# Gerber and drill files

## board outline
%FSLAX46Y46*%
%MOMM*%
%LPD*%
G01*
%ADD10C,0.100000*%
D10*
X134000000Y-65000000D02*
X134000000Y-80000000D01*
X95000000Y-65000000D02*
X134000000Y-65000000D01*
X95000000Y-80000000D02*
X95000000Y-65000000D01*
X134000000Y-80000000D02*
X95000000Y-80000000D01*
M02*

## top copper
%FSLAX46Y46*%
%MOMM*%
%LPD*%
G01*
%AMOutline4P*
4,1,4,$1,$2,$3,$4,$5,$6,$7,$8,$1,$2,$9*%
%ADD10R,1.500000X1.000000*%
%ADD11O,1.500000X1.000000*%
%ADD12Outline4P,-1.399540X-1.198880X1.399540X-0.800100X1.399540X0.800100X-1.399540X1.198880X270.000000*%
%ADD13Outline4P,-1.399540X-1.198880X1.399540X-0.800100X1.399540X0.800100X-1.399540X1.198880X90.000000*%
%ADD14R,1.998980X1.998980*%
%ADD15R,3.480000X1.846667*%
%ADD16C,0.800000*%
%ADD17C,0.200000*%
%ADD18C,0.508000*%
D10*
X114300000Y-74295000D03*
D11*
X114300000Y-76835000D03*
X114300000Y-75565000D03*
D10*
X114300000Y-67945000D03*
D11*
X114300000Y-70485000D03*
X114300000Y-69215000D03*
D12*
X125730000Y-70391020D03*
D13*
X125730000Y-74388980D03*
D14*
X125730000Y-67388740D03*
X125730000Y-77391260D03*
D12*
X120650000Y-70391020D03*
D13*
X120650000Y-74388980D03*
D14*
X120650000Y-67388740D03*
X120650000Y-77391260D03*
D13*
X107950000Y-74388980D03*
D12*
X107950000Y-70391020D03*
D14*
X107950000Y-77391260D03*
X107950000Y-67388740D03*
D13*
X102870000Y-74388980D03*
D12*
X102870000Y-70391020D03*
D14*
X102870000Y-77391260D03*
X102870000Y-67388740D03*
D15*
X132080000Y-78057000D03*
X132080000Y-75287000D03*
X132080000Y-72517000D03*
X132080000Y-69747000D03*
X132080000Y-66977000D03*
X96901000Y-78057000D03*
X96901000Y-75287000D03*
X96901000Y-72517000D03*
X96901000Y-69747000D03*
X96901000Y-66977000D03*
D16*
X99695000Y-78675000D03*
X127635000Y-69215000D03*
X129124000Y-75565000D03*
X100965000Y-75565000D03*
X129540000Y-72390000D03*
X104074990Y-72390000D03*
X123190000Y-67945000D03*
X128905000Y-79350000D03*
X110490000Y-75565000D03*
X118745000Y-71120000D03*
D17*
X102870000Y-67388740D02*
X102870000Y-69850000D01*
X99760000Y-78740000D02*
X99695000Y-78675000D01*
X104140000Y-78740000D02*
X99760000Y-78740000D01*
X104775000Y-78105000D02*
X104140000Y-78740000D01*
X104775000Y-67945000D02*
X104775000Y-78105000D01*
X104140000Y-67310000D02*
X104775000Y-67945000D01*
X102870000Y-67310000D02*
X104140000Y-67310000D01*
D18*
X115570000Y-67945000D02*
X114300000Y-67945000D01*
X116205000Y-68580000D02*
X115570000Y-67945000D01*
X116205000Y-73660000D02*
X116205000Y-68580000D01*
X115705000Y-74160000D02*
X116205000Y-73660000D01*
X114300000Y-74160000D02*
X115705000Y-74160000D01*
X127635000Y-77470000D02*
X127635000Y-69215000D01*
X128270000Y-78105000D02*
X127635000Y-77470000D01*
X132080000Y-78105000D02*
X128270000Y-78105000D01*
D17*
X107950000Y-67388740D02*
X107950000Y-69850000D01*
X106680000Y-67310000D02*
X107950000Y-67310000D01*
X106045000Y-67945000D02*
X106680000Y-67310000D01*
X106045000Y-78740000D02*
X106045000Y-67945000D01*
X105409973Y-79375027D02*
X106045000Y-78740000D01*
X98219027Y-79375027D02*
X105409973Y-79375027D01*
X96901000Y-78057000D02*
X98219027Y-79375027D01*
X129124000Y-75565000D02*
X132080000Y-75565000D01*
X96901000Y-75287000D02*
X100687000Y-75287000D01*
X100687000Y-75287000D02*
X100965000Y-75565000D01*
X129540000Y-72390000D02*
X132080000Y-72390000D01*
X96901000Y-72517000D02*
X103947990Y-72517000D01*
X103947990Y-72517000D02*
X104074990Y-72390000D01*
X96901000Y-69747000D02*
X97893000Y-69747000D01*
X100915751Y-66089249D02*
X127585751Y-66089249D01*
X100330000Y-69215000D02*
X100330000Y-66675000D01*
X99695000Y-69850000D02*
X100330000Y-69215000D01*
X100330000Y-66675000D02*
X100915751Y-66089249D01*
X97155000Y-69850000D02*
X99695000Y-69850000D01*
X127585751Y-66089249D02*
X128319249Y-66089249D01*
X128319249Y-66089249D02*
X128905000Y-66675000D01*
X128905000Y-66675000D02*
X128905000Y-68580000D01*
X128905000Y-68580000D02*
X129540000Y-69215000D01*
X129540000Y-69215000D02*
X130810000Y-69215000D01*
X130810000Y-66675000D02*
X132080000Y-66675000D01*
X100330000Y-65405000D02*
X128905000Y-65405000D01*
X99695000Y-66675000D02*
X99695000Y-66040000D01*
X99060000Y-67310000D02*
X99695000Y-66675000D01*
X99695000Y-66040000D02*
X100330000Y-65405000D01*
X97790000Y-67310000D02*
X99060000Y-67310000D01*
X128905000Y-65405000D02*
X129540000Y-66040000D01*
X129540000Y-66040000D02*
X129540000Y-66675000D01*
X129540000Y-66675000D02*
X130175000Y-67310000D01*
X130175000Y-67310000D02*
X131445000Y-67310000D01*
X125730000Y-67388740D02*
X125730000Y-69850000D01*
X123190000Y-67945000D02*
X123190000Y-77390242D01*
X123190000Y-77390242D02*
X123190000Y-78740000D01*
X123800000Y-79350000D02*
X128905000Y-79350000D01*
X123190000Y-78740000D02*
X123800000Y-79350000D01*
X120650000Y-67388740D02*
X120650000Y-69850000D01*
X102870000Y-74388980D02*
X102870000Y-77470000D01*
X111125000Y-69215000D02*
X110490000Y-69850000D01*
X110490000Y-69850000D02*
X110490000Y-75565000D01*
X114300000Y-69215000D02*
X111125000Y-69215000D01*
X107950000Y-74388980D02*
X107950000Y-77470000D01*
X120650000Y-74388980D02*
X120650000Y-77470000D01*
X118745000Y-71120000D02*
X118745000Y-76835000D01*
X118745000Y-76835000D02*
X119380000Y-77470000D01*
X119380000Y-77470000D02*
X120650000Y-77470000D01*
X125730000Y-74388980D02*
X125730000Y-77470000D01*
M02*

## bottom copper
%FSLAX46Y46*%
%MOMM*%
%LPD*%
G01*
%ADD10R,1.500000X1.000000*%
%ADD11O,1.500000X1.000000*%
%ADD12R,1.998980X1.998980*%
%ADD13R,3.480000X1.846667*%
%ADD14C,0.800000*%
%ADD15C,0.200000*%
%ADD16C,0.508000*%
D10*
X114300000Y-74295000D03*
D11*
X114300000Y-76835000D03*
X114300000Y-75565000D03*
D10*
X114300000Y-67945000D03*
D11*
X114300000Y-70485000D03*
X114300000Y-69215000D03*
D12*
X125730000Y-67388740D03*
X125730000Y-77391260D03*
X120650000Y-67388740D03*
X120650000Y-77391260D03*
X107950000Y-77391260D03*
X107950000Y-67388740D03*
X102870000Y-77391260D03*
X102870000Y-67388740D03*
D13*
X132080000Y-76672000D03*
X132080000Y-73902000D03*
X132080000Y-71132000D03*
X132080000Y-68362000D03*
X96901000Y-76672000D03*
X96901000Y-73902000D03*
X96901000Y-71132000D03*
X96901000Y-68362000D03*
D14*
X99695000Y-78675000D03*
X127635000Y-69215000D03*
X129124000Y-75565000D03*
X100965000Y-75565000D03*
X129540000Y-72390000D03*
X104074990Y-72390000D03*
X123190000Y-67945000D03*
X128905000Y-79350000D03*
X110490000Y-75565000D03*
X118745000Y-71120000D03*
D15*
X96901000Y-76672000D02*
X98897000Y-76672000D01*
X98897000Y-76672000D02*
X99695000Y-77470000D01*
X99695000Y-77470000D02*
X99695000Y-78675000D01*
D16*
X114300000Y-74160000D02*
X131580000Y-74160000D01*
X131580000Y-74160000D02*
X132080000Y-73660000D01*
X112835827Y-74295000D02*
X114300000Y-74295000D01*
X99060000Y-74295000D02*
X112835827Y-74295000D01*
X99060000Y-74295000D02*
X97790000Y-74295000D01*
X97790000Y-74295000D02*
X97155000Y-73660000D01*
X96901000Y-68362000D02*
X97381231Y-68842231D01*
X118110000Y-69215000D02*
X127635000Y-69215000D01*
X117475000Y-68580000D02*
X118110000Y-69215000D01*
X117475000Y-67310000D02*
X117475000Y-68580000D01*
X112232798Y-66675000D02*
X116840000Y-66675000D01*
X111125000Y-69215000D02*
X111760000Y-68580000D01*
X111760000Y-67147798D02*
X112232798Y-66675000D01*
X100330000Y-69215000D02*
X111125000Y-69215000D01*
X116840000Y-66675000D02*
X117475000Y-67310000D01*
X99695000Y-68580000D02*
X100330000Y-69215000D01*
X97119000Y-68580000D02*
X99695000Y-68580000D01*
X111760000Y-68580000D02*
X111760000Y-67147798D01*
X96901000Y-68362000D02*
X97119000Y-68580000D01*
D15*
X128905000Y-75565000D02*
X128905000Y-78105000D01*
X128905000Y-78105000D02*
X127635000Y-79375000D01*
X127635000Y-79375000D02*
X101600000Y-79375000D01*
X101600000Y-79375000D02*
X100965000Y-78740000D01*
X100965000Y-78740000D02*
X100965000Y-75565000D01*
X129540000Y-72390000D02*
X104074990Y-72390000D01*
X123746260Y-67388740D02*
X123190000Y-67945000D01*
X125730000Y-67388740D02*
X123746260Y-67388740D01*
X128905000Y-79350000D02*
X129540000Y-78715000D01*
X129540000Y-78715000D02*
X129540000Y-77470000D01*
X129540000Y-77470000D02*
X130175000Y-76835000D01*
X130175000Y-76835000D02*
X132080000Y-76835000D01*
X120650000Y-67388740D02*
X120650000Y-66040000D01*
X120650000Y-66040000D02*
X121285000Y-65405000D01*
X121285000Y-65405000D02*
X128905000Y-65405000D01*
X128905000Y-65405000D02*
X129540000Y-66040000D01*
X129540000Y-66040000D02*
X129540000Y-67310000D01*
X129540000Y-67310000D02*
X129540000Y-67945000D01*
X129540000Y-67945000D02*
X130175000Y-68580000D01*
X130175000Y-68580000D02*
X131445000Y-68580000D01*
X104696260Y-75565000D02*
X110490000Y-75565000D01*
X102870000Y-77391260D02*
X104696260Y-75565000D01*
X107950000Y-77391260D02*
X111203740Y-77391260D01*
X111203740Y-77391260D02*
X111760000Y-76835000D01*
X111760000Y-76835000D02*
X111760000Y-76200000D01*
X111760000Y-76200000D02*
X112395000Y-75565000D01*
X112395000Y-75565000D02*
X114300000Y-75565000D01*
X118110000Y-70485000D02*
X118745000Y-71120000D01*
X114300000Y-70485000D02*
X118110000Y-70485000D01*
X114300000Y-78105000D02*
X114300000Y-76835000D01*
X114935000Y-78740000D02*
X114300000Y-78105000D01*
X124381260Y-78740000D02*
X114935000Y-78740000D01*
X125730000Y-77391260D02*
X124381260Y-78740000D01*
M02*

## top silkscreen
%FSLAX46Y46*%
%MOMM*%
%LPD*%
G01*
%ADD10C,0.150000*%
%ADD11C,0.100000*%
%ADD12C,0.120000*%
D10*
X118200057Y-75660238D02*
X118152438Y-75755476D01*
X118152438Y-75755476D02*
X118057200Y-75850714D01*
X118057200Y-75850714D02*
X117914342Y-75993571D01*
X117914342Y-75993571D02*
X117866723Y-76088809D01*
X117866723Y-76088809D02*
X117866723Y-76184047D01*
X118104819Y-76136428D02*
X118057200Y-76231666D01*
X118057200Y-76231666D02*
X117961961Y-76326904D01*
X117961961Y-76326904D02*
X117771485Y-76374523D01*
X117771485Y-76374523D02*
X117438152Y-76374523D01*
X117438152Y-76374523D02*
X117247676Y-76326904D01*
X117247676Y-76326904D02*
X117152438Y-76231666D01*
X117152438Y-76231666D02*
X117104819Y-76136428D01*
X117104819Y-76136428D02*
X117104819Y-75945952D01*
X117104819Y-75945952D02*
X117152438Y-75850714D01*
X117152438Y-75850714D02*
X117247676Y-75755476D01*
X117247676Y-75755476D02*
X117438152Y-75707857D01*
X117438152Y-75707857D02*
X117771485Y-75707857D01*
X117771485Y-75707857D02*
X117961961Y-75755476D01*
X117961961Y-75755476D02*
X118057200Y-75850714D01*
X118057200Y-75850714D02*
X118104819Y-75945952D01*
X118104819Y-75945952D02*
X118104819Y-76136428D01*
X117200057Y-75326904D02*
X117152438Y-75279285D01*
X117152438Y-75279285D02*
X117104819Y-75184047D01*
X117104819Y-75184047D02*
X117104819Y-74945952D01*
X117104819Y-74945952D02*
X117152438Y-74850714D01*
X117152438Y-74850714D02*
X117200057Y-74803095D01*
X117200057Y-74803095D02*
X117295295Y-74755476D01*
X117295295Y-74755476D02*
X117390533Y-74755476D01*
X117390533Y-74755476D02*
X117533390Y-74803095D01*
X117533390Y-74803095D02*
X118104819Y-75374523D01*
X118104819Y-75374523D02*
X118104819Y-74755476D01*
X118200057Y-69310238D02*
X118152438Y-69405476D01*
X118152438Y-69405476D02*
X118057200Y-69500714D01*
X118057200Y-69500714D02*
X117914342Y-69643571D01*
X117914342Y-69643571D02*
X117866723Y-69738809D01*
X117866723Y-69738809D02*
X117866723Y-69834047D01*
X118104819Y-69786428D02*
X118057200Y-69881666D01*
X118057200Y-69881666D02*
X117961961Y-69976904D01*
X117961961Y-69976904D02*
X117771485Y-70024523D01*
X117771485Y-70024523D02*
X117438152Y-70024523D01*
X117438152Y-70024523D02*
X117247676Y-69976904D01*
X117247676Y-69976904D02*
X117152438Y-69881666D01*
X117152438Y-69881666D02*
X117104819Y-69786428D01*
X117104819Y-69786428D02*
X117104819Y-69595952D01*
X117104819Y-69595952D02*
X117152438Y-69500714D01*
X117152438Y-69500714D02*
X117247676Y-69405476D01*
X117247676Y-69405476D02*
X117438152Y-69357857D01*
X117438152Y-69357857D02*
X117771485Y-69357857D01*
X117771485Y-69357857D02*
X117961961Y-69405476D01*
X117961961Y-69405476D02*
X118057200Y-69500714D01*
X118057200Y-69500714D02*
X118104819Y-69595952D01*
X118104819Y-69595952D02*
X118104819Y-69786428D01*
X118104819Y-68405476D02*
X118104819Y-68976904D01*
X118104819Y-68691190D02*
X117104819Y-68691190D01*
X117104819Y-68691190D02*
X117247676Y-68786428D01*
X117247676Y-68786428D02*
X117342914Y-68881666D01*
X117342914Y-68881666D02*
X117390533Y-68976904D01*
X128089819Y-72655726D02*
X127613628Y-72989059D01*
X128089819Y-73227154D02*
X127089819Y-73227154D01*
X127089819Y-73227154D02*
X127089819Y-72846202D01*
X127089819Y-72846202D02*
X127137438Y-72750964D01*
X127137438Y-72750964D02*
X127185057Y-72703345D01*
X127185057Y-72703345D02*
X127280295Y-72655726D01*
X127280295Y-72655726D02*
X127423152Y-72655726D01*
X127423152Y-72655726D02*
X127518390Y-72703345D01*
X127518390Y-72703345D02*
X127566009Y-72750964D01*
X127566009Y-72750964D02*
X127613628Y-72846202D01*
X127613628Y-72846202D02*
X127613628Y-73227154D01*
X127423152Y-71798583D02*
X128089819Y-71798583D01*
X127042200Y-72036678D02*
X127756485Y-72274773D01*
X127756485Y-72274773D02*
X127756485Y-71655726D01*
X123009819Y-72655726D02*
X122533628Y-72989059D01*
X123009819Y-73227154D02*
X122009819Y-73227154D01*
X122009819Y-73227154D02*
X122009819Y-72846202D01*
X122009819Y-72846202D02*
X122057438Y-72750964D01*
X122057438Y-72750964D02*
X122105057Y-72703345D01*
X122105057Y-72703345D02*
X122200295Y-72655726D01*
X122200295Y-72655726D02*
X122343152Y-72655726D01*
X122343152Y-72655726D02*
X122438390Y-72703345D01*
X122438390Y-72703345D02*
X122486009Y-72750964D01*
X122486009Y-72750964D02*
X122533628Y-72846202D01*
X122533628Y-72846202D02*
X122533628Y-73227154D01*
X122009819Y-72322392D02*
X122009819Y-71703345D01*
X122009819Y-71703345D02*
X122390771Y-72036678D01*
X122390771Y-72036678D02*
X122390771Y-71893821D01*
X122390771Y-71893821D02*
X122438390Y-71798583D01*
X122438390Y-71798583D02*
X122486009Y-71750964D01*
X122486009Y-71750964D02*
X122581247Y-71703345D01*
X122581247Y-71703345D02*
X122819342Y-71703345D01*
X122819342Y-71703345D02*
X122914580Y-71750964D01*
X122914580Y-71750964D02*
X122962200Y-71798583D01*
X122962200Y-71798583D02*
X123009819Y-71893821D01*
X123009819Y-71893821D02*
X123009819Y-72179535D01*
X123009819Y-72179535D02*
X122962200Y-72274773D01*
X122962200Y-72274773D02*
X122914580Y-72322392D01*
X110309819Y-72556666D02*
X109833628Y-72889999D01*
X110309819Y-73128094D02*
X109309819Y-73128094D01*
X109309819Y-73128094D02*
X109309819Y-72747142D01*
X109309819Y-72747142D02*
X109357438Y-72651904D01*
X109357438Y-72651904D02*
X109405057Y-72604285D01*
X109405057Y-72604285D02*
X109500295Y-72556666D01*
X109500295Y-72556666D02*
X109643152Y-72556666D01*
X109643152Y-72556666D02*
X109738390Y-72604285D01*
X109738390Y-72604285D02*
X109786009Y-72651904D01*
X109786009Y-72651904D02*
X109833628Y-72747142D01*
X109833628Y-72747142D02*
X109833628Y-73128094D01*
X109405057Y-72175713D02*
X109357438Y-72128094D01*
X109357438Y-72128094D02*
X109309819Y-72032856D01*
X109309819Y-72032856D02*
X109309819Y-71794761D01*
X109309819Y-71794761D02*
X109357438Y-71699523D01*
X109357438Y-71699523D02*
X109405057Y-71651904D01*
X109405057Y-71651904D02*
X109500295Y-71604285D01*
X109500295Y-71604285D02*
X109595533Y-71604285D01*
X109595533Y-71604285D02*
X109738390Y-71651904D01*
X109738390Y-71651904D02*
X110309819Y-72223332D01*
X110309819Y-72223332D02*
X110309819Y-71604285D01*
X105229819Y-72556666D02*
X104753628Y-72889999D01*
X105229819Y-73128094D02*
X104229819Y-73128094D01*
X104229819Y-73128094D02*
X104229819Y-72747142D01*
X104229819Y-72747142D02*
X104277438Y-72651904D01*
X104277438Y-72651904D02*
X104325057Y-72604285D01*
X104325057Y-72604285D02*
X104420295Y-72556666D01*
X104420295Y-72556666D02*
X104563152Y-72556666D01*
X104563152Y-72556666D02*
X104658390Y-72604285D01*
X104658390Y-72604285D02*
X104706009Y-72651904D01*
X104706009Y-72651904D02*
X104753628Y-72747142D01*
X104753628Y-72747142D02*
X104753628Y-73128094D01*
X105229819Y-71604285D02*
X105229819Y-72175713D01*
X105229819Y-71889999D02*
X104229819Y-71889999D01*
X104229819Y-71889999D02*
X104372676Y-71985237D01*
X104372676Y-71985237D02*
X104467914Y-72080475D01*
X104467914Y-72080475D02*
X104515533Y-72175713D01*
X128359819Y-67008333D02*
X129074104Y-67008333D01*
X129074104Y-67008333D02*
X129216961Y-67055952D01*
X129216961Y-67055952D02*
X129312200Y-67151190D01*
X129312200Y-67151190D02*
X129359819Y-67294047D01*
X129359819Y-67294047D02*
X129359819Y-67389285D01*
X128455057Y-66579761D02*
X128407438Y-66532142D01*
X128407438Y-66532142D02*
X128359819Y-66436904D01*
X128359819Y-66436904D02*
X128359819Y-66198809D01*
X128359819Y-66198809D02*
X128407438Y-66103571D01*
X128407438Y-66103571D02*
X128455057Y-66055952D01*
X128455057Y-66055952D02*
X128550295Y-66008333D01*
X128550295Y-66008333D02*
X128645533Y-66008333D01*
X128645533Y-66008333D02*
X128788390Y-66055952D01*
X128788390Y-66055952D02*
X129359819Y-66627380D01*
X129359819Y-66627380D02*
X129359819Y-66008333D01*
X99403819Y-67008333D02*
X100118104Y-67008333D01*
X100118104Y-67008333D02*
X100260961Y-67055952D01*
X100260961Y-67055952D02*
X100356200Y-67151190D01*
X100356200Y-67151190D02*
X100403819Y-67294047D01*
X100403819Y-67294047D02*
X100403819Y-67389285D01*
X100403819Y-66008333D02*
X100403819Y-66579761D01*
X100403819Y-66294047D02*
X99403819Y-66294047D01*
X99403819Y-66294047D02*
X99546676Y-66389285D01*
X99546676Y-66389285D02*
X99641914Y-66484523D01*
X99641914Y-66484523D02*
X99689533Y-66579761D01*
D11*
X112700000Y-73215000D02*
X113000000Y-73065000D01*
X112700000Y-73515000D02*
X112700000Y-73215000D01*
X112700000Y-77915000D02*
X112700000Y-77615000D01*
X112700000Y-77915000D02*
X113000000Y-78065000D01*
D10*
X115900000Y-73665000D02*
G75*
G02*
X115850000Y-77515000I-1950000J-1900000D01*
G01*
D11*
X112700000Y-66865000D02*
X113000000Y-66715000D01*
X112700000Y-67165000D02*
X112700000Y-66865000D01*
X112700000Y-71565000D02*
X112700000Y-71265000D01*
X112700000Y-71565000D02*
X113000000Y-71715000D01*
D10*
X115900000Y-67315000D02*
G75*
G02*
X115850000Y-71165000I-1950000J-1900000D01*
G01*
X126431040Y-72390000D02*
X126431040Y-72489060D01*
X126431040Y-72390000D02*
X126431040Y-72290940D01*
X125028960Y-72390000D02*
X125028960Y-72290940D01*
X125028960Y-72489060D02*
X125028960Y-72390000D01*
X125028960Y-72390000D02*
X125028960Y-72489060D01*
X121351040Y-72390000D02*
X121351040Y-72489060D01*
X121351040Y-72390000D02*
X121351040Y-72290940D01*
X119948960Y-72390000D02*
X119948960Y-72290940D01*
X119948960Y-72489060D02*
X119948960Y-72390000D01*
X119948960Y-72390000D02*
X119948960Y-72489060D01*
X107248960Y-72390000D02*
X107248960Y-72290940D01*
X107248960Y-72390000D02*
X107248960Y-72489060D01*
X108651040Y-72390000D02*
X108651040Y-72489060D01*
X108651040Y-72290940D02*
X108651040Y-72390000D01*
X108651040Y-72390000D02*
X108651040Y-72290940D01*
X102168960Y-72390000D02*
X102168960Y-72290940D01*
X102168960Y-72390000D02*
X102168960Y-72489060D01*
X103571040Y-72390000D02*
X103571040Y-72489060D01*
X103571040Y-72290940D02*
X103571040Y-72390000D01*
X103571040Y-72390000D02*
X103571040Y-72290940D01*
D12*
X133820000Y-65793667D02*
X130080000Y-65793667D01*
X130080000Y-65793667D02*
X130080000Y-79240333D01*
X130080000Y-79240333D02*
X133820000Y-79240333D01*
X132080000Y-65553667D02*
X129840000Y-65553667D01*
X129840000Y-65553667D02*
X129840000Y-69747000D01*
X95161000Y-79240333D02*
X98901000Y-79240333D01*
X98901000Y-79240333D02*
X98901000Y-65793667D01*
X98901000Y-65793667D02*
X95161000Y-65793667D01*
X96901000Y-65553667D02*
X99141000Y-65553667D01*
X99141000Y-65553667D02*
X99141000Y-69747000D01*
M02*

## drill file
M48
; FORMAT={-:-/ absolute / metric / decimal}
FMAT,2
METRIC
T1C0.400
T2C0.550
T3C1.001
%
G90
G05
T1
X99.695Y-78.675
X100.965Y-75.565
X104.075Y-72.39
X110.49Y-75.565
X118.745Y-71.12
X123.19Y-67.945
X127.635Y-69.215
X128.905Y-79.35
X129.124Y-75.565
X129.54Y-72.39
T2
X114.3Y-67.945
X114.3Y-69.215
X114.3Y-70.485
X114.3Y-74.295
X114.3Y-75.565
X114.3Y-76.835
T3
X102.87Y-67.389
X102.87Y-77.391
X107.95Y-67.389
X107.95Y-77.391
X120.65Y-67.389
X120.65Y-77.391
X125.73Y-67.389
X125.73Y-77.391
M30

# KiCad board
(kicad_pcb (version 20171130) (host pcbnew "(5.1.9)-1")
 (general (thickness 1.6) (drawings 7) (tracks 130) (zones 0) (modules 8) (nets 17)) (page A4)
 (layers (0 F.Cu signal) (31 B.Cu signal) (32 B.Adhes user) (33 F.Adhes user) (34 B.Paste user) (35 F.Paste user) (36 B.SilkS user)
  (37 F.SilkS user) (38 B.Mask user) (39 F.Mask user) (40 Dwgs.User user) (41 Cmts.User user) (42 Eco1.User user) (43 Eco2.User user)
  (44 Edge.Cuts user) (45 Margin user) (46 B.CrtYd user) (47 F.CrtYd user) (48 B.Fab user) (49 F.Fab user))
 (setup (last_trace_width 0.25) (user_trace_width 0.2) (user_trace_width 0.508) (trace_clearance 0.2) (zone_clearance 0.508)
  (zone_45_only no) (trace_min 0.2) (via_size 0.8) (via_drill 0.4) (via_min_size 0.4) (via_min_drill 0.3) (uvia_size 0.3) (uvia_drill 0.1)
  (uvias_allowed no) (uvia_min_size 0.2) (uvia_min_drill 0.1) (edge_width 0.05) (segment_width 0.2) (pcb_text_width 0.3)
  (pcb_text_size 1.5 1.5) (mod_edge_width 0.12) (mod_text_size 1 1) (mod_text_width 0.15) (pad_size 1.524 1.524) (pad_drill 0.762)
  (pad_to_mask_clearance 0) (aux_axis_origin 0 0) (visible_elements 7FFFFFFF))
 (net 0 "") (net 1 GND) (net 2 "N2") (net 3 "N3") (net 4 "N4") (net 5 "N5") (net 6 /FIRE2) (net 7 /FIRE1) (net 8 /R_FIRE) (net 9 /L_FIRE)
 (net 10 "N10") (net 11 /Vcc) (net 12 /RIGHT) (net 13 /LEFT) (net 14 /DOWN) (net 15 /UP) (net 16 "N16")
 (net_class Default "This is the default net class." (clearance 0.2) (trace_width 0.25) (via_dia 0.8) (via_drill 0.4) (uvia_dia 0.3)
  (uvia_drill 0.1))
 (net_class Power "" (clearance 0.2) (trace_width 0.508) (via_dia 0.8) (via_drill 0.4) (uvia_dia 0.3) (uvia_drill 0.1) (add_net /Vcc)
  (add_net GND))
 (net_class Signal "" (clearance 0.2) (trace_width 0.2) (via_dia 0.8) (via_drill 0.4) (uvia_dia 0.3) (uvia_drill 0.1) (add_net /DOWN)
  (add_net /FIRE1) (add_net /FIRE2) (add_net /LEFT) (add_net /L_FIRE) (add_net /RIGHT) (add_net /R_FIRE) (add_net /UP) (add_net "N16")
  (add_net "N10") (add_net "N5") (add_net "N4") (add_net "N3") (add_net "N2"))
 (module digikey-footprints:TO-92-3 (layer F.Cu) (at 114.3 74.295 270)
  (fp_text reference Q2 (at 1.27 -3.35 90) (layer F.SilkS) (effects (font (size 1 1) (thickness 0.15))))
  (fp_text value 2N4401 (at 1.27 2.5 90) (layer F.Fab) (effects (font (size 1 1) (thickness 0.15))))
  (fp_line (start -1.08 1.6) (end -1.23 1.3) (layer F.SilkS) (width 0.1))
  (fp_line (start -0.78 1.6) (end -1.08 1.6) (layer F.SilkS) (width 0.1))
  (fp_line (start 3.62 1.6) (end 3.32 1.6) (layer F.SilkS) (width 0.1))
  (fp_line (start 3.62 1.6) (end 3.77 1.3) (layer F.SilkS) (width 0.1))
  (fp_arc (start 1.27 0.35) (end -0.63 -1.6) (angle 90) (layer F.SilkS) (width 0.15))
  (pad 1 thru_hole rect (at 0 0 90) (size 1 1.5) (drill 0.55) (layers *.Cu *.Mask) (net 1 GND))
  (pad 3 thru_hole oval (at 2.54 0 90) (size 1 1.5) (drill 0.55) (layers *.Cu *.Mask) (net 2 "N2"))
  (pad 2 thru_hole oval (at 1.27 0 90) (size 1 1.5) (drill 0.55) (layers *.Cu *.Mask) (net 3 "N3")))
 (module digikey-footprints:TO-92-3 (layer F.Cu) (at 114.3 67.945 270)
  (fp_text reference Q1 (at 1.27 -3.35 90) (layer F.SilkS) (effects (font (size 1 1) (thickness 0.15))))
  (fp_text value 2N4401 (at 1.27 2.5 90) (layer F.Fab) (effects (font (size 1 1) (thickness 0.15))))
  (fp_line (start -1.08 1.6) (end -1.23 1.3) (layer F.SilkS) (width 0.1))
  (fp_line (start -0.78 1.6) (end -1.08 1.6) (layer F.SilkS) (width 0.1))
  (fp_line (start 3.62 1.6) (end 3.32 1.6) (layer F.SilkS) (width 0.1))
  (fp_line (start 3.62 1.6) (end 3.77 1.3) (layer F.SilkS) (width 0.1))
  (fp_arc (start 1.27 0.35) (end -0.63 -1.6) (angle 90) (layer F.SilkS) (width 0.15))
  (pad 1 thru_hole rect (at 0 0 90) (size 1 1.5) (drill 0.55) (layers *.Cu *.Mask) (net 1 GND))
  (pad 3 thru_hole oval (at 2.54 0 90) (size 1 1.5) (drill 0.55) (layers *.Cu *.Mask) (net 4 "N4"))
  (pad 2 thru_hole oval (at 1.27 0 90) (size 1 1.5) (drill 0.55) (layers *.Cu *.Mask) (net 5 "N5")))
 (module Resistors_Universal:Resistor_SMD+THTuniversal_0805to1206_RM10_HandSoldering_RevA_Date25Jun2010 (layer F.Cu) (at 125.73 72.39 270)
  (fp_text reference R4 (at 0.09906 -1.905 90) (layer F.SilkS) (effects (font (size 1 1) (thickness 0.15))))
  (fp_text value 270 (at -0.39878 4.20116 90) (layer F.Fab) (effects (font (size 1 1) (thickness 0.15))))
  (fp_line (start 0 -0.70104) (end 0.09906 -0.70104) (layer F.SilkS) (width 0.15))
  (fp_line (start 0 -0.70104) (end -0.09906 -0.70104) (layer F.SilkS) (width 0.15))
  (fp_line (start 0 0.70104) (end -0.09906 0.70104) (layer F.SilkS) (width 0.15))
  (fp_line (start 0.09906 0.70104) (end 0 0.70104) (layer F.SilkS) (width 0.15))
  (fp_line (start 0 0.70104) (end 0.09906 0.70104) (layer F.SilkS) (width 0.15))
  (pad 1 smd trapezoid (at -1.99898 0 270) (size 2.79908 1.99898) (rect_delta 0.39878 0) (layers F.Cu F.Paste F.Mask) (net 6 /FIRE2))
  (pad 2 smd trapezoid (at 1.99898 0 90) (size 2.79908 1.99898) (rect_delta 0.39878 0) (layers F.Cu F.Paste F.Mask) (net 2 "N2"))
  (pad 1 thru_hole rect (at -5.00126 0 90) (size 1.99898 1.99898) (drill 1.00076) (layers *.Cu *.Mask) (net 6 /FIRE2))
  (pad 2 thru_hole rect (at 5.00126 0 90) (size 1.99898 1.99898) (drill 1.00076) (layers *.Cu *.Mask) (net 2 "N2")))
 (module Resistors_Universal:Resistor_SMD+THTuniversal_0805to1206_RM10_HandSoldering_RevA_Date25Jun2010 (layer F.Cu) (at 120.65 72.39 270)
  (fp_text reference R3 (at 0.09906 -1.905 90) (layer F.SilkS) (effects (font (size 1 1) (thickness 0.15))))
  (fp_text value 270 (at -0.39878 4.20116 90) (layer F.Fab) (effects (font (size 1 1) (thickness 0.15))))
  (fp_line (start 0 -0.70104) (end 0.09906 -0.70104) (layer F.SilkS) (width 0.15))
  (fp_line (start 0 -0.70104) (end -0.09906 -0.70104) (layer F.SilkS) (width 0.15))
  (fp_line (start 0 0.70104) (end -0.09906 0.70104) (layer F.SilkS) (width 0.15))
  (fp_line (start 0.09906 0.70104) (end 0 0.70104) (layer F.SilkS) (width 0.15))
  (fp_line (start 0 0.70104) (end 0.09906 0.70104) (layer F.SilkS) (width 0.15))
  (pad 1 smd trapezoid (at -1.99898 0 270) (size 2.79908 1.99898) (rect_delta 0.39878 0) (layers F.Cu F.Paste F.Mask) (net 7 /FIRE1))
  (pad 2 smd trapezoid (at 1.99898 0 90) (size 2.79908 1.99898) (rect_delta 0.39878 0) (layers F.Cu F.Paste F.Mask) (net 4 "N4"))
  (pad 1 thru_hole rect (at -5.00126 0 90) (size 1.99898 1.99898) (drill 1.00076) (layers *.Cu *.Mask) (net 7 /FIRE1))
  (pad 2 thru_hole rect (at 5.00126 0 90) (size 1.99898 1.99898) (drill 1.00076) (layers *.Cu *.Mask) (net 4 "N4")))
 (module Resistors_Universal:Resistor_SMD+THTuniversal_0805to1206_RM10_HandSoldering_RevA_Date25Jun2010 (layer F.Cu) (at 107.95 72.39 90)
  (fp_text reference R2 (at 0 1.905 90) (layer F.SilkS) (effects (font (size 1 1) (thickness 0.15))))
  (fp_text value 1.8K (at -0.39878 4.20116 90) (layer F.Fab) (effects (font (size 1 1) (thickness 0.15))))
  (fp_line (start 0 -0.70104) (end 0.09906 -0.70104) (layer F.SilkS) (width 0.15))
  (fp_line (start 0 -0.70104) (end -0.09906 -0.70104) (layer F.SilkS) (width 0.15))
  (fp_line (start 0 0.70104) (end -0.09906 0.70104) (layer F.SilkS) (width 0.15))
  (fp_line (start 0.09906 0.70104) (end 0 0.70104) (layer F.SilkS) (width 0.15))
  (fp_line (start 0 0.70104) (end 0.09906 0.70104) (layer F.SilkS) (width 0.15))
  (pad 1 smd trapezoid (at -1.99898 0 90) (size 2.79908 1.99898) (rect_delta 0.39878 0) (layers F.Cu F.Paste F.Mask) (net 3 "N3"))
  (pad 2 smd trapezoid (at 1.99898 0 270) (size 2.79908 1.99898) (rect_delta 0.39878 0) (layers F.Cu F.Paste F.Mask) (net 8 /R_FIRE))
  (pad 1 thru_hole rect (at -5.00126 0 270) (size 1.99898 1.99898) (drill 1.00076) (layers *.Cu *.Mask) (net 3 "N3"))
  (pad 2 thru_hole rect (at 5.00126 0 270) (size 1.99898 1.99898) (drill 1.00076) (layers *.Cu *.Mask) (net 8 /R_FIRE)))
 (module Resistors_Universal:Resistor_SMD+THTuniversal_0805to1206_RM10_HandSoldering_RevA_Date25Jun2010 (layer F.Cu) (at 102.87 72.39 90)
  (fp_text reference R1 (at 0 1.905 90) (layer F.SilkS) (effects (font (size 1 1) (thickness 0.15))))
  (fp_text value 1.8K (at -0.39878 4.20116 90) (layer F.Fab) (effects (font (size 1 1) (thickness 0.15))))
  (fp_line (start 0 -0.70104) (end 0.09906 -0.70104) (layer F.SilkS) (width 0.15))
  (fp_line (start 0 -0.70104) (end -0.09906 -0.70104) (layer F.SilkS) (width 0.15))
  (fp_line (start 0 0.70104) (end -0.09906 0.70104) (layer F.SilkS) (width 0.15))
  (fp_line (start 0.09906 0.70104) (end 0 0.70104) (layer F.SilkS) (width 0.15))
  (fp_line (start 0 0.70104) (end 0.09906 0.70104) (layer F.SilkS) (width 0.15))
  (pad 1 smd trapezoid (at -1.99898 0 90) (size 2.79908 1.99898) (rect_delta 0.39878 0) (layers F.Cu F.Paste F.Mask) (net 5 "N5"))
  (pad 2 smd trapezoid (at 1.99898 0 270) (size 2.79908 1.99898) (rect_delta 0.39878 0) (layers F.Cu F.Paste F.Mask) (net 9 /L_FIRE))
  (pad 1 thru_hole rect (at -5.00126 0 270) (size 1.99898 1.99898) (drill 1.00076) (layers *.Cu *.Mask) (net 5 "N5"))
  (pad 2 thru_hole rect (at 5.00126 0 270) (size 1.99898 1.99898) (drill 1.00076) (layers *.Cu *.Mask) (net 9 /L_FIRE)))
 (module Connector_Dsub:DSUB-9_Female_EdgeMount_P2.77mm (layer F.Cu) (at 132.08 72.517 90)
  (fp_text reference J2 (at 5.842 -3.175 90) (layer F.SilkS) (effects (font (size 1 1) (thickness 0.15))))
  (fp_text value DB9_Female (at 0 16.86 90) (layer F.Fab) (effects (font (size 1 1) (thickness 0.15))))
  (fp_line (start 6.723333 1.74) (end 6.723333 -2) (layer F.SilkS) (width 0.12))
  (fp_line (start 6.723333 -2) (end -6.723333 -2) (layer F.SilkS) (width 0.12))
  (fp_line (start -6.723333 -2) (end -6.723333 1.74) (layer F.SilkS) (width 0.12))
  (fp_line (start 6.963333 0) (end 6.963333 -2.24) (layer F.SilkS) (width 0.12))
  (fp_line (start 6.963333 -2.24) (end 2.77 -2.24) (layer F.SilkS) (width 0.12))
  (pad 9 smd rect (at -4.155 0 90) (size 1.846667 3.48) (layers B.Cu B.Paste B.Mask) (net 6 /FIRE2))
  (pad 8 smd rect (at -1.385 0 90) (size 1.846667 3.48) (layers B.Cu B.Paste B.Mask) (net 1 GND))
  (pad 7 smd rect (at 1.385 0 90) (size 1.846667 3.48) (layers B.Cu B.Paste B.Mask) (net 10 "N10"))
  (pad 6 smd rect (at 4.155 0 90) (size 1.846667 3.48) (layers B.Cu B.Paste B.Mask) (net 7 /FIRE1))
  (pad 5 smd rect (at -5.54 0 90) (size 1.846667 3.48) (layers F.Cu F.Paste F.Mask) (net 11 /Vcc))
  (pad 4 smd rect (at -2.77 0 90) (size 1.846667 3.48) (layers F.Cu F.Paste F.Mask) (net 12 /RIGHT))
  (pad 3 smd rect (at 0 0 90) (size 1.846667 3.48) (layers F.Cu F.Paste F.Mask) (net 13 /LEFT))
  (pad 2 smd rect (at 2.77 0 90) (size 1.846667 3.48) (layers F.Cu F.Paste F.Mask) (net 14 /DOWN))
  (pad 1 smd rect (at 5.54 0 90) (size 1.846667 3.48) (layers F.Cu F.Paste F.Mask) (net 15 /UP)))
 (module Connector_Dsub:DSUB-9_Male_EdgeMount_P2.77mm (layer F.Cu) (at 96.901 72.517 270)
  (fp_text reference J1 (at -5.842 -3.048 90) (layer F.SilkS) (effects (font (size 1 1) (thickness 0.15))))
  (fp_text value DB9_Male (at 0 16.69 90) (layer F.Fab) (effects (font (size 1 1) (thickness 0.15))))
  (fp_line (start 6.723333 1.74) (end 6.723333 -2) (layer F.SilkS) (width 0.12))
  (fp_line (start 6.723333 -2) (end -6.723333 -2) (layer F.SilkS) (width 0.12))
  (fp_line (start -6.723333 -2) (end -6.723333 1.74) (layer F.SilkS) (width 0.12))
  (fp_line (start -6.963333 0) (end -6.963333 -2.24) (layer F.SilkS) (width 0.12))
  (fp_line (start -6.963333 -2.24) (end -2.77 -2.24) (layer F.SilkS) (width 0.12))
  (pad 9 smd rect (at 4.155 0 270) (size 1.846667 3.48) (layers B.Cu B.Paste B.Mask) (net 9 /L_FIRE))
  (pad 8 smd rect (at 1.385 0 270) (size 1.846667 3.48) (layers B.Cu B.Paste B.Mask) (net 1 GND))
  (pad 7 smd rect (at -1.385 0 270) (size 1.846667 3.48) (layers B.Cu B.Paste B.Mask) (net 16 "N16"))
  (pad 6 smd rect (at -4.155 0 270) (size 1.846667 3.48) (layers B.Cu B.Paste B.Mask) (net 11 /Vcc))
  (pad 5 smd rect (at 5.54 0 270) (size 1.846667 3.48) (layers F.Cu F.Paste F.Mask) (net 8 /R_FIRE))
  (pad 4 smd rect (at 2.77 0 270) (size 1.846667 3.48) (layers F.Cu F.Paste F.Mask) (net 12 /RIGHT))
  (pad 3 smd rect (at 0 0 270) (size 1.846667 3.48) (layers F.Cu F.Paste F.Mask) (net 13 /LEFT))
  (pad 2 smd rect (at -2.77 0 270) (size 1.846667 3.48) (layers F.Cu F.Paste F.Mask) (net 14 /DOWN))
  (pad 1 smd rect (at -5.54 0 270) (size 1.846667 3.48) (layers F.Cu F.Paste F.Mask) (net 15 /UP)))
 (gr_line (start 134 65) (end 134 80) (layer Edge.Cuts) (width 0.1))
 (gr_line (start 95 65) (end 134 65) (layer Edge.Cuts) (width 0.1))
 (gr_line (start 95 80) (end 95 65) (layer Edge.Cuts) (width 0.1))
 (gr_line (start 134 80) (end 95 80) (layer Edge.Cuts) (width 0.1))
 (segment (start 102.87 67.38874) (end 102.87 69.85) (width 0.2) (layer F.Cu) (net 9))
 (segment (start 96.901 76.672) (end 98.897 76.672) (width 0.2) (layer B.Cu) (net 9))
 (segment (start 98.897 76.672) (end 99.695 77.47) (width 0.2) (layer B.Cu) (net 9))
 (segment (start 99.695 77.47) (end 99.695 78.675) (width 0.2) (layer B.Cu) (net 9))
 (via (at 99.695 78.675) (size 0.8) (drill 0.4) (layers F.Cu B.Cu) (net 9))
 (segment (start 99.76 78.74) (end 99.695 78.675) (width 0.2) (layer F.Cu) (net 9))
 (segment (start 104.14 78.74) (end 99.76 78.74) (width 0.2) (layer F.Cu) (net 9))
 (segment (start 104.775 78.105) (end 104.14 78.74) (width 0.2) (layer F.Cu) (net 9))
 (segment (start 104.775 67.945) (end 104.775 78.105) (width 0.2) (layer F.Cu) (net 9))
 (segment (start 104.14 67.31) (end 104.775 67.945) (width 0.2) (layer F.Cu) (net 9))
 (segment (start 102.87 67.31) (end 104.14 67.31) (width 0.2) (layer F.Cu) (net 9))
 (segment (start 114.3 74.16) (end 131.58 74.16) (width 0.508) (layer B.Cu) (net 1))
 (segment (start 131.58 74.16) (end 132.08 73.66) (width 0.508) (layer B.Cu) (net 1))
 (segment (start 112.835827 74.295) (end 114.3 74.295) (width 0.508) (layer B.Cu) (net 1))
 (segment (start 99.06 74.295) (end 112.835827 74.295) (width 0.508) (layer B.Cu) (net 1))
 (segment (start 99.06 74.295) (end 97.79 74.295) (width 0.508) (layer B.Cu) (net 1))
 (segment (start 97.79 74.295) (end 97.155 73.66) (width 0.508) (layer B.Cu) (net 1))
 (segment (start 115.57 67.945) (end 114.3 67.945) (width 0.508) (layer F.Cu) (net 1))
 (segment (start 116.205 68.58) (end 115.57 67.945) (width 0.508) (layer F.Cu) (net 1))
 (segment (start 116.205 73.66) (end 116.205 68.58) (width 0.508) (layer F.Cu) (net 1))
 (segment (start 115.705 74.16) (end 116.205 73.66) (width 0.508) (layer F.Cu) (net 1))
 (segment (start 114.3 74.16) (end 115.705 74.16) (width 0.508) (layer F.Cu) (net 1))
 (segment (start 96.901 68.362) (end 97.381231 68.842231) (width 0.508) (layer B.Cu) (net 11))
 (via (at 127.635 69.215) (size 0.8) (drill 0.4) (layers F.Cu B.Cu) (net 11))
 (segment (start 127.635 77.47) (end 127.635 69.215) (width 0.508) (layer F.Cu) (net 11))
 (segment (start 128.27 78.105) (end 127.635 77.47) (width 0.508) (layer F.Cu) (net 11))
 (segment (start 132.08 78.105) (end 128.27 78.105) (width 0.508) (layer F.Cu) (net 11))
 (segment (start 118.11 69.215) (end 127.635 69.215) (width 0.508) (layer B.Cu) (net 11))
 (segment (start 117.475 68.58) (end 118.11 69.215) (width 0.508) (layer B.Cu) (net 11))
 (segment (start 117.475 67.31) (end 117.475 68.58) (width 0.508) (layer B.Cu) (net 11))
 (segment (start 112.232798 66.675) (end 116.84 66.675) (width 0.508) (layer B.Cu) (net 11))
 (segment (start 111.125 69.215) (end 111.76 68.58) (width 0.508) (layer B.Cu) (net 11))
 (segment (start 111.76 67.147798) (end 112.232798 66.675) (width 0.508) (layer B.Cu) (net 11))
 (segment (start 100.33 69.215) (end 111.125 69.215) (width 0.508) (layer B.Cu) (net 11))
 (segment (start 116.84 66.675) (end 117.475 67.31) (width 0.508) (layer B.Cu) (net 11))
 (segment (start 99.695 68.58) (end 100.33 69.215) (width 0.508) (layer B.Cu) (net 11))
 (segment (start 97.119 68.58) (end 99.695 68.58) (width 0.508) (layer B.Cu) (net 11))
 (segment (start 111.76 68.58) (end 111.76 67.147798) (width 0.508) (layer B.Cu) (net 11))
 (segment (start 96.901 68.362) (end 97.119 68.58) (width 0.508) (layer B.Cu) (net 11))
 (segment (start 107.95 67.38874) (end 107.95 69.85) (width 0.2) (layer F.Cu) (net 8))
 (segment (start 106.68 67.31) (end 107.95 67.31) (width 0.2) (layer F.Cu) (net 8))
 (segment (start 106.045 67.945) (end 106.68 67.31) (width 0.2) (layer F.Cu) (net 8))
 (segment (start 106.045 78.74) (end 106.045 67.945) (width 0.2) (layer F.Cu) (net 8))
 (segment (start 105.409973 79.375027) (end 106.045 78.74) (width 0.2) (layer F.Cu) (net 8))
 (segment (start 98.219027 79.375027) (end 105.409973 79.375027) (width 0.2) (layer F.Cu) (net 8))
 (segment (start 96.901 78.057) (end 98.219027 79.375027) (width 0.2) (layer F.Cu) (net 8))
 (via (at 129.124 75.565) (size 0.8) (drill 0.4) (layers F.Cu B.Cu) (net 12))
 (segment (start 129.124 75.565) (end 132.08 75.565) (width 0.2) (layer F.Cu) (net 12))
 (via (at 100.965 75.565) (size 0.8) (drill 0.4) (layers F.Cu B.Cu) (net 12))
 (segment (start 96.901 75.287) (end 100.687 75.287) (width 0.2) (layer F.Cu) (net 12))
 (segment (start 100.687 75.287) (end 100.965 75.565) (width 0.2) (layer F.Cu) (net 12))
 (segment (start 128.905 75.565) (end 128.905 78.105) (width 0.2) (layer B.Cu) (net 12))
 (segment (start 128.905 78.105) (end 127.635 79.375) (width 0.2) (layer B.Cu) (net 12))
 (segment (start 127.635 79.375) (end 101.6 79.375) (width 0.2) (layer B.Cu) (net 12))
 (segment (start 101.6 79.375) (end 100.965 78.74) (width 0.2) (layer B.Cu) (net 12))
 (segment (start 100.965 78.74) (end 100.965 75.565) (width 0.2) (layer B.Cu) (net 12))
 (via (at 129.54 72.39) (size 0.8) (drill 0.4) (layers F.Cu B.Cu) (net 13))
 (segment (start 129.54 72.39) (end 132.08 72.39) (width 0.2) (layer F.Cu) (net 13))
 (segment (start 96.901 72.517) (end 103.94799 72.517) (width 0.2) (layer F.Cu) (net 13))
 (via (at 104.07499 72.39) (size 0.8) (drill 0.4) (layers F.Cu B.Cu) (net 13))
 (segment (start 129.54 72.39) (end 104.07499 72.39) (width 0.2) (layer B.Cu) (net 13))
 (segment (start 103.94799 72.517) (end 104.07499 72.39) (width 0.2) (layer F.Cu) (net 13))
 (segment (start 96.901 69.747) (end 97.893 69.747) (width 0.2) (layer F.Cu) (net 14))
 (segment (start 100.915751 66.089249) (end 127.585751 66.089249) (width 0.2) (layer F.Cu) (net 14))
 (segment (start 100.33 69.215) (end 100.33 66.675) (width 0.2) (layer F.Cu) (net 14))
 (segment (start 99.695 69.85) (end 100.33 69.215) (width 0.2) (layer F.Cu) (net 14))
 (segment (start 100.33 66.675) (end 100.915751 66.089249) (width 0.2) (layer F.Cu) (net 14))
 (segment (start 97.155 69.85) (end 99.695 69.85) (width 0.2) (layer F.Cu) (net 14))
 (segment (start 127.585751 66.089249) (end 128.319249 66.089249) (width 0.2) (layer F.Cu) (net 14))
 (segment (start 128.319249 66.089249) (end 128.905 66.675) (width 0.2) (layer F.Cu) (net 14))
 (segment (start 128.905 66.675) (end 128.905 68.58) (width 0.2) (layer F.Cu) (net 14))
 (segment (start 128.905 68.58) (end 129.54 69.215) (width 0.2) (layer F.Cu) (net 14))
 (segment (start 129.54 69.215) (end 130.81 69.215) (width 0.2) (layer F.Cu) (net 14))
 (segment (start 130.81 66.675) (end 132.08 66.675) (width 0.2) (layer F.Cu) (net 15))
 (segment (start 100.33 65.405) (end 128.905 65.405) (width 0.2) (layer F.Cu) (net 15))
 (segment (start 99.695 66.675) (end 99.695 66.04) (width 0.2) (layer F.Cu) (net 15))
 (segment (start 99.06 67.31) (end 99.695 66.675) (width 0.2) (layer F.Cu) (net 15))
 (segment (start 99.695 66.04) (end 100.33 65.405) (width 0.2) (layer F.Cu) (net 15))
 (segment (start 97.79 67.31) (end 99.06 67.31) (width 0.2) (layer F.Cu) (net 15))
 (segment (start 128.905 65.405) (end 129.54 66.04) (width 0.2) (layer F.Cu) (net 15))
 (segment (start 129.54 66.04) (end 129.54 66.675) (width 0.2) (layer F.Cu) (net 15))
 (segment (start 129.54 66.675) (end 130.175 67.31) (width 0.2) (layer F.Cu) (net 15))
 (segment (start 130.175 67.31) (end 131.445 67.31) (width 0.2) (layer F.Cu) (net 15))
 (segment (start 125.73 67.38874) (end 125.73 69.85) (width 0.2) (layer F.Cu) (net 6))
 (via (at 123.19 67.945) (size 0.8) (drill 0.4) (layers F.Cu B.Cu) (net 6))
 (segment (start 123.74626 67.38874) (end 123.19 67.945) (width 0.2) (layer B.Cu) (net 6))
 (segment (start 125.73 67.38874) (end 123.74626 67.38874) (width 0.2) (layer B.Cu) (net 6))
 (segment (start 123.19 67.945) (end 123.19 77.390242) (width 0.2) (layer F.Cu) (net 6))
 (segment (start 123.19 77.390242) (end 123.19 78.74) (width 0.2) (layer F.Cu) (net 6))
 (segment (start 123.8 79.35) (end 128.905 79.35) (width 0.2) (layer F.Cu) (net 6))
 (via (at 128.905 79.35) (size 0.8) (drill 0.4) (layers F.Cu B.Cu) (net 6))
 (segment (start 123.19 78.74) (end 123.8 79.35) (width 0.2) (layer F.Cu) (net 6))
 (segment (start 128.905 79.35) (end 129.54 78.715) (width 0.2) (layer B.Cu) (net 6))
 (segment (start 129.54 78.715) (end 129.54 77.47) (width 0.2) (layer B.Cu) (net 6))
 (segment (start 129.54 77.47) (end 130.175 76.835) (width 0.2) (layer B.Cu) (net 6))
 (segment (start 130.175 76.835) (end 132.08 76.835) (width 0.2) (layer B.Cu) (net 6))
 (segment (start 120.65 67.38874) (end 120.65 69.85) (width 0.2) (layer F.Cu) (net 7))
 (segment (start 120.65 67.38874) (end 120.65 66.04) (width 0.2) (layer B.Cu) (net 7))
 (segment (start 120.65 66.04) (end 121.285 65.405) (width 0.2) (layer B.Cu) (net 7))
 (segment (start 121.285 65.405) (end 128.905 65.405) (width 0.2) (layer B.Cu) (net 7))
 (segment (start 128.905 65.405) (end 129.54 66.04) (width 0.2) (layer B.Cu) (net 7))
 (segment (start 129.54 66.04) (end 129.54 67.31) (width 0.2) (layer B.Cu) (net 7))
 (segment (start 129.54 67.31) (end 129.54 67.945) (width 0.2) (layer B.Cu) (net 7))
 (segment (start 129.54 67.945) (end 130.175 68.58) (width 0.2) (layer B.Cu) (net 7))
 (segment (start 130.175 68.58) (end 131.445 68.58) (width 0.2) (layer B.Cu) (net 7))
 (segment (start 102.87 74.38898) (end 102.87 77.47) (width 0.2) (layer F.Cu) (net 5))
 (segment (start 104.69626 75.565) (end 110.49 75.565) (width 0.2) (layer B.Cu) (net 5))
 (segment (start 102.87 77.39126) (end 104.69626 75.565) (width 0.2) (layer B.Cu) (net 5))
 (via (at 110.49 75.565) (size 0.8) (drill 0.4) (layers F.Cu B.Cu) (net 5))
 (segment (start 111.125 69.215) (end 110.49 69.85) (width 0.2) (layer F.Cu) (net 5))
 (segment (start 110.49 69.85) (end 110.49 75.565) (width 0.2) (layer F.Cu) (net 5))
 (segment (start 114.3 69.215) (end 111.125 69.215) (width 0.2) (layer F.Cu) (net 5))
 (segment (start 107.95 74.38898) (end 107.95 77.47) (width 0.2) (layer F.Cu) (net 3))
 (segment (start 107.95 77.39126) (end 111.20374 77.39126) (width 0.2) (layer B.Cu) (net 3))
 (segment (start 111.20374 77.39126) (end 111.76 76.835) (width 0.2) (layer B.Cu) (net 3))
 (segment (start 111.76 76.835) (end 111.76 76.2) (width 0.2) (layer B.Cu) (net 3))
 (segment (start 111.76 76.2) (end 112.395 75.565) (width 0.2) (layer B.Cu) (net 3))
 (segment (start 112.395 75.565) (end 114.3 75.565) (width 0.2) (layer B.Cu) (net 3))
 (segment (start 120.65 74.38898) (end 120.65 77.47) (width 0.2) (layer F.Cu) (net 4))
 (via (at 118.745 71.12) (size 0.8) (drill 0.4) (layers F.Cu B.Cu) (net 4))
 (segment (start 118.745 71.12) (end 118.745 76.835) (width 0.2) (layer F.Cu) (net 4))
 (segment (start 118.745 76.835) (end 119.38 77.47) (width 0.2) (layer F.Cu) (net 4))
 (segment (start 119.38 77.47) (end 120.65 77.47) (width 0.2) (layer F.Cu) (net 4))
 (segment (start 118.11 70.485) (end 118.745 71.12) (width 0.2) (layer B.Cu) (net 4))
 (segment (start 114.3 70.485) (end 118.11 70.485) (width 0.2) (layer B.Cu) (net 4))
 (segment (start 125.73 74.38898) (end 125.73 77.47) (width 0.2) (layer F.Cu) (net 2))
 (segment (start 114.3 78.105) (end 114.3 76.835) (width 0.2) (layer B.Cu) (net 2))
 (segment (start 114.935 78.74) (end 114.3 78.105) (width 0.2) (layer B.Cu) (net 2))
 (segment (start 124.38126 78.74) (end 114.935 78.74) (width 0.2) (layer B.Cu) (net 2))
 (segment (start 125.73 77.39126) (end 124.38126 78.74) (width 0.2) (layer B.Cu) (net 2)))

